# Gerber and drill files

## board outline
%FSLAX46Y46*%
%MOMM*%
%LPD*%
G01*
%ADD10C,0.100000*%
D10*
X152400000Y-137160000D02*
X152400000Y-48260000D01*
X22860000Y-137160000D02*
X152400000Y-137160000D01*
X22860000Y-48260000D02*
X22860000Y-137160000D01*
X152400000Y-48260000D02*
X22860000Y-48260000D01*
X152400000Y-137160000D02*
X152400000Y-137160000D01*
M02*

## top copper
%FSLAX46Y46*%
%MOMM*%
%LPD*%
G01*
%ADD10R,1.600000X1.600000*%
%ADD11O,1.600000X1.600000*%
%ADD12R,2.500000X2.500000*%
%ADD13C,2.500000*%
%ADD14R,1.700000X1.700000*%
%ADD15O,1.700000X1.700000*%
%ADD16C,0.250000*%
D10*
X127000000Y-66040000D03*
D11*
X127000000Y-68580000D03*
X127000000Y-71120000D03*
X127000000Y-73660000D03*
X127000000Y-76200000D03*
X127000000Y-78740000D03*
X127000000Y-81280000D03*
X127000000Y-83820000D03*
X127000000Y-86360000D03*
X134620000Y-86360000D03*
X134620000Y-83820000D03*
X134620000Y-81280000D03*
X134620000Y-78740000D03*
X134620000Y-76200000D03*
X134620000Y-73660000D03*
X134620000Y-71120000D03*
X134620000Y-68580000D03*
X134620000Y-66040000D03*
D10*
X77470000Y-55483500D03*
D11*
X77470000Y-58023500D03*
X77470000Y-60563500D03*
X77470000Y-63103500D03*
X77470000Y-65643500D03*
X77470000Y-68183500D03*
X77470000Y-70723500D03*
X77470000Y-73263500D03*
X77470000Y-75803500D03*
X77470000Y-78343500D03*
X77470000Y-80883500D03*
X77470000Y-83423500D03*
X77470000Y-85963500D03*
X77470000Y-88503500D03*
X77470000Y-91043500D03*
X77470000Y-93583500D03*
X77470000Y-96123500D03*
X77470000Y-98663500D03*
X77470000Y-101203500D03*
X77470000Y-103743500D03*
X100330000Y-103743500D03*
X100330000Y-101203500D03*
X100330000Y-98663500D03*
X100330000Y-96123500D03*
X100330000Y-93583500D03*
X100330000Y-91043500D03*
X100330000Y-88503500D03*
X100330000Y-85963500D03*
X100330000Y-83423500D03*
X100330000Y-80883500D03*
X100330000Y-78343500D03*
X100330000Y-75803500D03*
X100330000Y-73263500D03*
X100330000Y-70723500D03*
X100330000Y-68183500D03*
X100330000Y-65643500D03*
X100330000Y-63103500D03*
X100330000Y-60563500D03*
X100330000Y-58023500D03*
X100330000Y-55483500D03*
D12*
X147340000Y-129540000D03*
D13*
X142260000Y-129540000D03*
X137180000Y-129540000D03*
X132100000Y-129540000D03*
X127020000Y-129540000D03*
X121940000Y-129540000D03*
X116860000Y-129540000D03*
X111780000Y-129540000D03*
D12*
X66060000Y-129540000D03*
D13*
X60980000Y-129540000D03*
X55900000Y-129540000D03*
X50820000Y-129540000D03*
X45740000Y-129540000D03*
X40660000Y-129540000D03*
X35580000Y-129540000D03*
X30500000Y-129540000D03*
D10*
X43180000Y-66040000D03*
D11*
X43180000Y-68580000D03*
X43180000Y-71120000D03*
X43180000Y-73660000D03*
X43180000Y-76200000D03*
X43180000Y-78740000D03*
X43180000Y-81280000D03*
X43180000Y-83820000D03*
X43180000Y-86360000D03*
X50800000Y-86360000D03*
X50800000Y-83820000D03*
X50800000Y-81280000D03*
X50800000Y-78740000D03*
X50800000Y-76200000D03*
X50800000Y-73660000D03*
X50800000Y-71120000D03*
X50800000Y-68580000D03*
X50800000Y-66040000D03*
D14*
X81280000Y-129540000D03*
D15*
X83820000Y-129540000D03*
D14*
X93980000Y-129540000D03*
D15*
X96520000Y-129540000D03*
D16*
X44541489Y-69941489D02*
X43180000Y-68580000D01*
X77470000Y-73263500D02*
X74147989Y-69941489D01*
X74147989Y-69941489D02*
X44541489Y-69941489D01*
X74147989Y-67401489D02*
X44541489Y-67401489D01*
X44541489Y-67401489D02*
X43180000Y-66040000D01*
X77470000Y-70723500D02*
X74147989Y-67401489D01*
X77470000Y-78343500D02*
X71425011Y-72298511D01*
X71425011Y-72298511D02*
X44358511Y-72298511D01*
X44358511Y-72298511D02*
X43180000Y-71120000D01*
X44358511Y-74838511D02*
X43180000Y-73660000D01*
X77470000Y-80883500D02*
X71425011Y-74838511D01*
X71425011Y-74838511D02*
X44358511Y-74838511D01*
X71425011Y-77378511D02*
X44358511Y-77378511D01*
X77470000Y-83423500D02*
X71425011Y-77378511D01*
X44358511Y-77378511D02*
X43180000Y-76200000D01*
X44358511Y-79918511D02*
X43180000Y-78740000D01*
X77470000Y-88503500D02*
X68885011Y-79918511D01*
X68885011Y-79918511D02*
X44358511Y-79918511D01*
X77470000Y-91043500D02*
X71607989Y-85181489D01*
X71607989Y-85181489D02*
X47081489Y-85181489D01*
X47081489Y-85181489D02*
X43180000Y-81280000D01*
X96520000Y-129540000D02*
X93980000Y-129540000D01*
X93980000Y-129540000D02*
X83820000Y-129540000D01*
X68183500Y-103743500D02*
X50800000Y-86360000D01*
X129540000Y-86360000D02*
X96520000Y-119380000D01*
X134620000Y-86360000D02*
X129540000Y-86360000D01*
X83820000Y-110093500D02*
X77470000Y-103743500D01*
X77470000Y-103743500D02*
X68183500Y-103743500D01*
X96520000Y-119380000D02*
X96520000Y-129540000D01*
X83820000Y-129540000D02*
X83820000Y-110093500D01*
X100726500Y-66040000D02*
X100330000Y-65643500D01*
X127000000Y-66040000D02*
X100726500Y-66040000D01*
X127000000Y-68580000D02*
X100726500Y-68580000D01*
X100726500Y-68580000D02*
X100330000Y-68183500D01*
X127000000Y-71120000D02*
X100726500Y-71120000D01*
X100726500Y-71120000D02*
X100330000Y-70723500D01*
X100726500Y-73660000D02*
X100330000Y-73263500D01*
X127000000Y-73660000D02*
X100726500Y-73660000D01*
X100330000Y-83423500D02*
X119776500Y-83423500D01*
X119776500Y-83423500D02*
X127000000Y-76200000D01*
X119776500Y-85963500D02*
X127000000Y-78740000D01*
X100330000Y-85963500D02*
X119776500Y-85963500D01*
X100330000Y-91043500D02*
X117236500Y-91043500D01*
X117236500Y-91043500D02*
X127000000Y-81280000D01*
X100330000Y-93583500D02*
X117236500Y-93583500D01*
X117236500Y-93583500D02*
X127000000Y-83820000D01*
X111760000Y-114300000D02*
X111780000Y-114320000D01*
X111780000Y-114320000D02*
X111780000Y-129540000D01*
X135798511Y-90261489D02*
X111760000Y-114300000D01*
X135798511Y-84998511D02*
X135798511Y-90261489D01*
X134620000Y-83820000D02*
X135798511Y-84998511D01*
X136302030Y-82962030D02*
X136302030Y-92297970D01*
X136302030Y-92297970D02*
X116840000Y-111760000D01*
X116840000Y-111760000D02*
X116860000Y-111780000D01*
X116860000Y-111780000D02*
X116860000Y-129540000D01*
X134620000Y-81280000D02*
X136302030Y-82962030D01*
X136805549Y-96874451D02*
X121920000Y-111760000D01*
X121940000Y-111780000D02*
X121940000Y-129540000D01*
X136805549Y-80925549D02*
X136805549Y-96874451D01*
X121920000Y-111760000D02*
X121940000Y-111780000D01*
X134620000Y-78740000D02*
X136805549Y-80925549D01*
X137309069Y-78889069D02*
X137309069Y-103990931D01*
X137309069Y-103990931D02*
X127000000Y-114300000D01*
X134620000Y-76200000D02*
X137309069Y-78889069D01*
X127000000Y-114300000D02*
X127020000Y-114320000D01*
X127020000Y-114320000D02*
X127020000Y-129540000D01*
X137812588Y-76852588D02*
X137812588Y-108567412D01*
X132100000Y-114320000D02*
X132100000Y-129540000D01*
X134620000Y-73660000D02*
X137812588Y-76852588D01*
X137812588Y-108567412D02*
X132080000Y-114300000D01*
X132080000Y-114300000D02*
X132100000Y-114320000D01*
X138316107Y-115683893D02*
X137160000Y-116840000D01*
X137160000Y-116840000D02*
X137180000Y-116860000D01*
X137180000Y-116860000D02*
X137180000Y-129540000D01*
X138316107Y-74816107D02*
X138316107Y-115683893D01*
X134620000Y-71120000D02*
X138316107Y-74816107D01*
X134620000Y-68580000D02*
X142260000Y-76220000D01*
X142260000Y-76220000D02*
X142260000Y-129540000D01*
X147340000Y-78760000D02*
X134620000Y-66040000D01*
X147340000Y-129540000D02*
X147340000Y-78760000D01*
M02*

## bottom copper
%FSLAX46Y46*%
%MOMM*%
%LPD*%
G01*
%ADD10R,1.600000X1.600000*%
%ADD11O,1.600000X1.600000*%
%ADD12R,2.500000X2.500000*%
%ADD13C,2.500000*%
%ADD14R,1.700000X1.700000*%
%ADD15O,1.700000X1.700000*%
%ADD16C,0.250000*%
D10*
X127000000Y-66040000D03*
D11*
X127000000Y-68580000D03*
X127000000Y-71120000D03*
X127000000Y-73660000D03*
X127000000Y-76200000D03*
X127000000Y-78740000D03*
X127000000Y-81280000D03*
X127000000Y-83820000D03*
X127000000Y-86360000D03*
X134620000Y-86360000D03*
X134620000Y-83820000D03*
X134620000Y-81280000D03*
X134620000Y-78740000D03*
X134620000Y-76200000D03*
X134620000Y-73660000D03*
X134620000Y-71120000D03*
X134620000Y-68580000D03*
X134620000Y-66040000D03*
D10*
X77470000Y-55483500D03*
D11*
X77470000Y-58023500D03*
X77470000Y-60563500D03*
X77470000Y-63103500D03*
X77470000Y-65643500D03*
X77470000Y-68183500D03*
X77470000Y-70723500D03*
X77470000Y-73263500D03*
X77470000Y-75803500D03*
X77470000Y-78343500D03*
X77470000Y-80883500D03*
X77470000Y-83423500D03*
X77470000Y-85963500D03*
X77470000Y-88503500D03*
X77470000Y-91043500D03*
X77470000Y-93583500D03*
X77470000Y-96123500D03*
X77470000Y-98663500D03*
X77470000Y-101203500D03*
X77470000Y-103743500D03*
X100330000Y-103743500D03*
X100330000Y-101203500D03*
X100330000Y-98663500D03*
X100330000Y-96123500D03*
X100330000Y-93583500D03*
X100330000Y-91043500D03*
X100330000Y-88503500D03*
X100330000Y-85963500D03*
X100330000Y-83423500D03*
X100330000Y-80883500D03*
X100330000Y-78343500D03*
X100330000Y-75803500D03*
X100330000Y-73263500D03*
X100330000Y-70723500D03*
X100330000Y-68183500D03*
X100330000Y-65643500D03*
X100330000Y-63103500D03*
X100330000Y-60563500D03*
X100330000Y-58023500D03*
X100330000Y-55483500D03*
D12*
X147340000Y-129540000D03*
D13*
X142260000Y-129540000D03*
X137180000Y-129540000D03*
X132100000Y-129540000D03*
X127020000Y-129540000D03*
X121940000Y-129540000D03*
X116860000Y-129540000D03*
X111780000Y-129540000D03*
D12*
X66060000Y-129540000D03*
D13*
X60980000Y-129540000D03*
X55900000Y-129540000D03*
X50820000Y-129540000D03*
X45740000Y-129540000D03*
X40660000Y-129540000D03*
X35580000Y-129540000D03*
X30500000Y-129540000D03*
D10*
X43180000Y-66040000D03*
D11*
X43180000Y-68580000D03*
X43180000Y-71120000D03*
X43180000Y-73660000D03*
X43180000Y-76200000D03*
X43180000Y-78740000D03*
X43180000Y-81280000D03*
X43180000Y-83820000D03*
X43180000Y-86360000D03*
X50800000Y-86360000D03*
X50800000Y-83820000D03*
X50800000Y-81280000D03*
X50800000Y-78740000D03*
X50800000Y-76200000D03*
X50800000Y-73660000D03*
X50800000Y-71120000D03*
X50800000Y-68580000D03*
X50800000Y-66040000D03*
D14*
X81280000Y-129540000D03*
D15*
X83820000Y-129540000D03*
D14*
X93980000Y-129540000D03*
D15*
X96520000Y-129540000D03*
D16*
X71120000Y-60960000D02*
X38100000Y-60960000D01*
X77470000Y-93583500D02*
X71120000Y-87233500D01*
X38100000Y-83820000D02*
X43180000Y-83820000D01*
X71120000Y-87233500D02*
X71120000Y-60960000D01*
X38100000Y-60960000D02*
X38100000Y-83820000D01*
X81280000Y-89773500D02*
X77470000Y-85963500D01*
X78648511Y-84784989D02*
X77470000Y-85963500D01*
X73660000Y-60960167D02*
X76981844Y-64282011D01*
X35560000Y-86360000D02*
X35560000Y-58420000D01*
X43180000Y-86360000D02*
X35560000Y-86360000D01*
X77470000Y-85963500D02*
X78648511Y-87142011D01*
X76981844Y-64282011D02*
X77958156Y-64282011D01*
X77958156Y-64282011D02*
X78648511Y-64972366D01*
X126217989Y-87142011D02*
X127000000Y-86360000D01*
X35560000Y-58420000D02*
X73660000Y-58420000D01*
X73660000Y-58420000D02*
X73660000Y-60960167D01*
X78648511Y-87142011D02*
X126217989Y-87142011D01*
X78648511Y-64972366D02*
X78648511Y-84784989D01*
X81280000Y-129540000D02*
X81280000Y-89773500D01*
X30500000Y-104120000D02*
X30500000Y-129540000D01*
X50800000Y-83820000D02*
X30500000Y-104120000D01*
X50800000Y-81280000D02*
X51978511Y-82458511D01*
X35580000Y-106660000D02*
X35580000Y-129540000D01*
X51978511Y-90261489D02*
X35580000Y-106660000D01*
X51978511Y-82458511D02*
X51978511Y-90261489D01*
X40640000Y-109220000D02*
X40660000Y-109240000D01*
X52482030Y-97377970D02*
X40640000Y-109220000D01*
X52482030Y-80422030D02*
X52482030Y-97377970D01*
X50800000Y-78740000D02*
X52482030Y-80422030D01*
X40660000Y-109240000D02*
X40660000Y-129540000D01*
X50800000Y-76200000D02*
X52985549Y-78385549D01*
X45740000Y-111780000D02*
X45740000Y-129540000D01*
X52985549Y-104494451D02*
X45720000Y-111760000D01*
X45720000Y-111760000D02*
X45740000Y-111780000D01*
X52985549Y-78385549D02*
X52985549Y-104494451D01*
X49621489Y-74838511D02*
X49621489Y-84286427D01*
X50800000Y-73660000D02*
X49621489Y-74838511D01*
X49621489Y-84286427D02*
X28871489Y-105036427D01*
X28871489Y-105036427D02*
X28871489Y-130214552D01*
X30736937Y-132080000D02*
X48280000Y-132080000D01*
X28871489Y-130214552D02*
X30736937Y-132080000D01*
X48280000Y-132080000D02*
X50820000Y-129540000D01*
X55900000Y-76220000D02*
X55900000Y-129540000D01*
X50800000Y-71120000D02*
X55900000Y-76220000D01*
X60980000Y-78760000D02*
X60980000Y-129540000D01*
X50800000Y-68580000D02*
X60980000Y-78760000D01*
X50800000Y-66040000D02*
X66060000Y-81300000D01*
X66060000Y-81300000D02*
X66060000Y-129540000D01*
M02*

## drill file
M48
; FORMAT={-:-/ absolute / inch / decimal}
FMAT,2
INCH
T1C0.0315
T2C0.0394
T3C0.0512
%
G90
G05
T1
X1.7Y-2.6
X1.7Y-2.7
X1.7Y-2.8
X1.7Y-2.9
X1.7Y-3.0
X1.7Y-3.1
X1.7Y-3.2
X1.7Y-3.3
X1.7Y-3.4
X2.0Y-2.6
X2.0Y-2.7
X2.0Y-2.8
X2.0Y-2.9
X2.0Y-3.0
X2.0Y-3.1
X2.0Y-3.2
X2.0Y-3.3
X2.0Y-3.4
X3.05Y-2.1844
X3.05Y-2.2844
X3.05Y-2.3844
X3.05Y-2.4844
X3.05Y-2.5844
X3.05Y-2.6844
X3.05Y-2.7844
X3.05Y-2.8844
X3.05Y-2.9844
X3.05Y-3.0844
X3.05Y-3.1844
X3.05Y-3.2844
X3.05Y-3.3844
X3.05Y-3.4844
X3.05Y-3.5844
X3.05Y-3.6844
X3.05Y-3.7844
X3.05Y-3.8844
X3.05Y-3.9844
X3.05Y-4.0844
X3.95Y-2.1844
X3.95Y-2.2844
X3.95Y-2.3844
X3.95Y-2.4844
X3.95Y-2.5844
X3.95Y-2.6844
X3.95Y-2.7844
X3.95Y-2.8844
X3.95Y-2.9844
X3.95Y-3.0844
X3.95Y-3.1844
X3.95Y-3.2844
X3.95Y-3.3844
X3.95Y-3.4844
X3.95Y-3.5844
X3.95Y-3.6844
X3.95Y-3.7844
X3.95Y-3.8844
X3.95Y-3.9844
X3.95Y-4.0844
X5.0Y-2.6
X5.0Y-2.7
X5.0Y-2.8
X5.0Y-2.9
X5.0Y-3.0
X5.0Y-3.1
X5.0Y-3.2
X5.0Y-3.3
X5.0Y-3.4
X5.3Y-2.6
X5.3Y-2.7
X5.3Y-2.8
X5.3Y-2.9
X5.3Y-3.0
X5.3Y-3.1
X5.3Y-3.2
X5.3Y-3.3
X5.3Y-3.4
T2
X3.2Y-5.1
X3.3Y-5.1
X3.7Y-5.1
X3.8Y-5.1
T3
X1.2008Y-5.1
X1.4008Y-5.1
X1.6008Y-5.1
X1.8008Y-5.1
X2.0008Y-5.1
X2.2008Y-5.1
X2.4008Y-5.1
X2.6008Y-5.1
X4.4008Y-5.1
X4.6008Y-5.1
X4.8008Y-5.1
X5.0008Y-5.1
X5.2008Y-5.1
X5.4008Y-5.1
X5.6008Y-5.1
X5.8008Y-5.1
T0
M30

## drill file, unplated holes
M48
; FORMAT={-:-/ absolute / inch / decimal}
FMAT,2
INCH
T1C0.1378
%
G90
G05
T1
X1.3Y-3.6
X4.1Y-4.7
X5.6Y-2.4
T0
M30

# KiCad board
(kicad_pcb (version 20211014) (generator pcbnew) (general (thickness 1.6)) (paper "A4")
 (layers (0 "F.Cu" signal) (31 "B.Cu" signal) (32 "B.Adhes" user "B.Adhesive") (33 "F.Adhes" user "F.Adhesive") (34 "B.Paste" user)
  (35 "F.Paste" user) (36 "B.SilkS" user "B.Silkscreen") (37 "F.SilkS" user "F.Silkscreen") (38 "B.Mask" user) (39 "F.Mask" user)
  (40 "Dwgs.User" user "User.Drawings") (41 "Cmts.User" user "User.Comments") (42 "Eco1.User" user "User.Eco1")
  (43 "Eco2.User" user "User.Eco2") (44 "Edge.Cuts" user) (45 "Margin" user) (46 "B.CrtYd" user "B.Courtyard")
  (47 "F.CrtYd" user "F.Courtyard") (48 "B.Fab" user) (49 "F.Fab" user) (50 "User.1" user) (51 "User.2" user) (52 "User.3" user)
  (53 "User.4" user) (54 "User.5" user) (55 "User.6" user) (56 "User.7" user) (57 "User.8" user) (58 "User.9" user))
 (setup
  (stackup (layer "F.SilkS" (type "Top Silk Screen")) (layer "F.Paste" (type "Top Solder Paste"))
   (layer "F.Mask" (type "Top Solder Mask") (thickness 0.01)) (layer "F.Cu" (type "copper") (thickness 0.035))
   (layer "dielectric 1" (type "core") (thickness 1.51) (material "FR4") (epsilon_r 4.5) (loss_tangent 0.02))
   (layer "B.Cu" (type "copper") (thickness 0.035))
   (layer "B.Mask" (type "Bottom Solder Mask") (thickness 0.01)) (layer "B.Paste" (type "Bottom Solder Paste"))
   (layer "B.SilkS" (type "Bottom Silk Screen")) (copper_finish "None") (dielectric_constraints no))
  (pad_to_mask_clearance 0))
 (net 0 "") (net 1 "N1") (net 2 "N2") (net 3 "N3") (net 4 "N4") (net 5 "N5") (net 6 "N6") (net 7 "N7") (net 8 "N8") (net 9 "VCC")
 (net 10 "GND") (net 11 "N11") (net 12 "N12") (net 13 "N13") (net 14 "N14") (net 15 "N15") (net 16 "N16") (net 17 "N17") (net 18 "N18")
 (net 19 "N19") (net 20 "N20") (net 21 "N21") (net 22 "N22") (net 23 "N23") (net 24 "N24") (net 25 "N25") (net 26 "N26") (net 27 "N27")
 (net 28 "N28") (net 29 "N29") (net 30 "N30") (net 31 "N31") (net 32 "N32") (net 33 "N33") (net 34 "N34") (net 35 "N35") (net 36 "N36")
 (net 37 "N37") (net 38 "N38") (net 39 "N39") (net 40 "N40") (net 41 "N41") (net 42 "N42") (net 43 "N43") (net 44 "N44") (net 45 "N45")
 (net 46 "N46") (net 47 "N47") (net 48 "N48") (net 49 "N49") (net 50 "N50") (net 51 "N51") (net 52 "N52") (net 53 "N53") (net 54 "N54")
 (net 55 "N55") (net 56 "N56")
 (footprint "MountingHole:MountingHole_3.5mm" (layer "F.Cu") (at 142.24 60.96)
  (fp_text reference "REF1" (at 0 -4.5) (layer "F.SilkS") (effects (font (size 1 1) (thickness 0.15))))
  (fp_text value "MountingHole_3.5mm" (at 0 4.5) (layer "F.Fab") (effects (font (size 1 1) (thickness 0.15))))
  (pad "" np_thru_hole circle (at 0 0) (size 3.5 3.5) (drill 3.5) (layers *.Cu *.Mask)))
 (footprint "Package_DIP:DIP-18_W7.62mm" (layer "F.Cu") (at 127 66.04)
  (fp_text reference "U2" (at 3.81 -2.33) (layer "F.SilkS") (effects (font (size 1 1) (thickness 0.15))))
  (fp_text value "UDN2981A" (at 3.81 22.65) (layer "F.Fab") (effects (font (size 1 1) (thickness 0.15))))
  (pad "1" thru_hole rect (at 0 0) (size 1.6 1.6) (drill 0.8) (layers *.Cu *.Mask) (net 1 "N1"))
  (pad "2" thru_hole oval (at 0 2.54) (size 1.6 1.6) (drill 0.8) (layers *.Cu *.Mask) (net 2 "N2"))
  (pad "3" thru_hole oval (at 0 5.08) (size 1.6 1.6) (drill 0.8) (layers *.Cu *.Mask) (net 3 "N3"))
  (pad "4" thru_hole oval (at 0 7.62) (size 1.6 1.6) (drill 0.8) (layers *.Cu *.Mask) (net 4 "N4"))
  (pad "5" thru_hole oval (at 0 10.16) (size 1.6 1.6) (drill 0.8) (layers *.Cu *.Mask) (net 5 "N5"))
  (pad "6" thru_hole oval (at 0 12.7) (size 1.6 1.6) (drill 0.8) (layers *.Cu *.Mask) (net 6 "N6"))
  (pad "7" thru_hole oval (at 0 15.24) (size 1.6 1.6) (drill 0.8) (layers *.Cu *.Mask) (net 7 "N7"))
  (pad "8" thru_hole oval (at 0 17.78) (size 1.6 1.6) (drill 0.8) (layers *.Cu *.Mask) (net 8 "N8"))
  (pad "9" thru_hole oval (at 0 20.32) (size 1.6 1.6) (drill 0.8) (layers *.Cu *.Mask) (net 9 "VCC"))
  (pad "10" thru_hole oval (at 7.62 20.32) (size 1.6 1.6) (drill 0.8) (layers *.Cu *.Mask) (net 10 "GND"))
  (pad "11" thru_hole oval (at 7.62 17.78) (size 1.6 1.6) (drill 0.8) (layers *.Cu *.Mask) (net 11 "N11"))
  (pad "12" thru_hole oval (at 7.62 15.24) (size 1.6 1.6) (drill 0.8) (layers *.Cu *.Mask) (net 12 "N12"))
  (pad "13" thru_hole oval (at 7.62 12.7) (size 1.6 1.6) (drill 0.8) (layers *.Cu *.Mask) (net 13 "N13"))
  (pad "14" thru_hole oval (at 7.62 10.16) (size 1.6 1.6) (drill 0.8) (layers *.Cu *.Mask) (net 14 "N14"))
  (pad "15" thru_hole oval (at 7.62 7.62) (size 1.6 1.6) (drill 0.8) (layers *.Cu *.Mask) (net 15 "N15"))
  (pad "16" thru_hole oval (at 7.62 5.08) (size 1.6 1.6) (drill 0.8) (layers *.Cu *.Mask) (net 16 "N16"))
  (pad "17" thru_hole oval (at 7.62 2.54) (size 1.6 1.6) (drill 0.8) (layers *.Cu *.Mask) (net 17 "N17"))
  (pad "18" thru_hole oval (at 7.62 0) (size 1.6 1.6) (drill 0.8) (layers *.Cu *.Mask) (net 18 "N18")))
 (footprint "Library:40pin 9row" (layer "F.Cu") (at 77.47 55.4835)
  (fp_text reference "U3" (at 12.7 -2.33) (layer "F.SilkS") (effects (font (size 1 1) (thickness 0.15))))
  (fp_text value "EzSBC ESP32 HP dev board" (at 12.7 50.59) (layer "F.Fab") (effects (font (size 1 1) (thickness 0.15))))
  (pad "1" thru_hole rect (at 0 0) (size 1.6 1.6) (drill 0.8) (layers *.Cu *.Mask) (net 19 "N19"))
  (pad "2" thru_hole oval (at 0 2.54) (size 1.6 1.6) (drill 0.8) (layers *.Cu *.Mask) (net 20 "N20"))
  (pad "3" thru_hole oval (at 0 5.08) (size 1.6 1.6) (drill 0.8) (layers *.Cu *.Mask) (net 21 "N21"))
  (pad "4" thru_hole oval (at 0 7.62) (size 1.6 1.6) (drill 0.8) (layers *.Cu *.Mask) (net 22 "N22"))
  (pad "5" thru_hole oval (at 0 10.16) (size 1.6 1.6) (drill 0.8) (layers *.Cu *.Mask) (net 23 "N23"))
  (pad "6" thru_hole oval (at 0 12.7) (size 1.6 1.6) (drill 0.8) (layers *.Cu *.Mask) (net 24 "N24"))
  (pad "7" thru_hole oval (at 0 15.24) (size 1.6 1.6) (drill 0.8) (layers *.Cu *.Mask) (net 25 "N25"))
  (pad "8" thru_hole oval (at 0 17.78) (size 1.6 1.6) (drill 0.8) (layers *.Cu *.Mask) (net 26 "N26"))
  (pad "9" thru_hole oval (at 0 20.32) (size 1.6 1.6) (drill 0.8) (layers *.Cu *.Mask) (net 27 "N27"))
  (pad "10" thru_hole oval (at 0 22.86) (size 1.6 1.6) (drill 0.8) (layers *.Cu *.Mask) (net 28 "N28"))
  (pad "11" thru_hole oval (at 0 25.4) (size 1.6 1.6) (drill 0.8) (layers *.Cu *.Mask) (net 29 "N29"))
  (pad "12" thru_hole oval (at 0 27.94) (size 1.6 1.6) (drill 0.8) (layers *.Cu *.Mask) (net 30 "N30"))
  (pad "13" thru_hole oval (at 0 30.48) (size 1.6 1.6) (drill 0.8) (layers *.Cu *.Mask) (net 9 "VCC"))
  (pad "14" thru_hole oval (at 0 33.02) (size 1.6 1.6) (drill 0.8) (layers *.Cu *.Mask) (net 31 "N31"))
  (pad "15" thru_hole oval (at 0 35.56) (size 1.6 1.6) (drill 0.8) (layers *.Cu *.Mask) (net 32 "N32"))
  (pad "16" thru_hole oval (at 0 38.1) (size 1.6 1.6) (drill 0.8) (layers *.Cu *.Mask) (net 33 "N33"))
  (pad "17" thru_hole oval (at 0 40.64) (size 1.6 1.6) (drill 0.8) (layers *.Cu *.Mask) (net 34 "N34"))
  (pad "18" thru_hole oval (at 0 43.18) (size 1.6 1.6) (drill 0.8) (layers *.Cu *.Mask) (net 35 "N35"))
  (pad "19" thru_hole oval (at 0 45.72) (size 1.6 1.6) (drill 0.8) (layers *.Cu *.Mask) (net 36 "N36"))
  (pad "20" thru_hole oval (at 0 48.26) (size 1.6 1.6) (drill 0.8) (layers *.Cu *.Mask) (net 10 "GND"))
  (pad "21" thru_hole oval (at 22.86 48.26) (size 1.6 1.6) (drill 0.8) (layers *.Cu *.Mask) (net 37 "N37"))
  (pad "22" thru_hole oval (at 22.86 45.72) (size 1.6 1.6) (drill 0.8) (layers *.Cu *.Mask) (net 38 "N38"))
  (pad "23" thru_hole oval (at 22.86 43.18) (size 1.6 1.6) (drill 0.8) (layers *.Cu *.Mask) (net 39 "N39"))
  (pad "24" thru_hole oval (at 22.86 40.64) (size 1.6 1.6) (drill 0.8) (layers *.Cu *.Mask) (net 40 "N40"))
  (pad "25" thru_hole oval (at 22.86 38.1) (size 1.6 1.6) (drill 0.8) (layers *.Cu *.Mask) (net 8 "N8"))
  (pad "26" thru_hole oval (at 22.86 35.56) (size 1.6 1.6) (drill 0.8) (layers *.Cu *.Mask) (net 7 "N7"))
  (pad "27" thru_hole oval (at 22.86 33.02) (size 1.6 1.6) (drill 0.8) (layers *.Cu *.Mask) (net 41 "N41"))
  (pad "28" thru_hole oval (at 22.86 30.48) (size 1.6 1.6) (drill 0.8) (layers *.Cu *.Mask) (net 6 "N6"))
  (pad "29" thru_hole oval (at 22.86 27.94) (size 1.6 1.6) (drill 0.8) (layers *.Cu *.Mask) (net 5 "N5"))
  (pad "30" thru_hole oval (at 22.86 25.4) (size 1.6 1.6) (drill 0.8) (layers *.Cu *.Mask) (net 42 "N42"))
  (pad "31" thru_hole oval (at 22.86 22.86) (size 1.6 1.6) (drill 0.8) (layers *.Cu *.Mask) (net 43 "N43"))
  (pad "32" thru_hole oval (at 22.86 20.32) (size 1.6 1.6) (drill 0.8) (layers *.Cu *.Mask) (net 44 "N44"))
  (pad "33" thru_hole oval (at 22.86 17.78) (size 1.6 1.6) (drill 0.8) (layers *.Cu *.Mask) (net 4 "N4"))
  (pad "34" thru_hole oval (at 22.86 15.24) (size 1.6 1.6) (drill 0.8) (layers *.Cu *.Mask) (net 3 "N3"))
  (pad "35" thru_hole oval (at 22.86 12.7) (size 1.6 1.6) (drill 0.8) (layers *.Cu *.Mask) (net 2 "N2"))
  (pad "36" thru_hole oval (at 22.86 10.16) (size 1.6 1.6) (drill 0.8) (layers *.Cu *.Mask) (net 1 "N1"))
  (pad "37" thru_hole oval (at 22.86 7.62) (size 1.6 1.6) (drill 0.8) (layers *.Cu *.Mask) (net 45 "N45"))
  (pad "38" thru_hole oval (at 22.86 5.08) (size 1.6 1.6) (drill 0.8) (layers *.Cu *.Mask) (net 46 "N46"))
  (pad "39" thru_hole oval (at 22.86 2.54) (size 1.6 1.6) (drill 0.8) (layers *.Cu *.Mask) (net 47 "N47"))
  (pad "40" thru_hole oval (at 22.86 0) (size 1.6 1.6) (drill 0.8) (layers *.Cu *.Mask) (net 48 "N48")))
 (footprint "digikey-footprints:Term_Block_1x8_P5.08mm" (layer "F.Cu") (at 147.34 129.54 180)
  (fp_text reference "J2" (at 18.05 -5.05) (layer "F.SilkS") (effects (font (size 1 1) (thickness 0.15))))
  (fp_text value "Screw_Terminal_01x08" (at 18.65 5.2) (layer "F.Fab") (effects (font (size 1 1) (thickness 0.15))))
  (pad "1" thru_hole rect locked (at 0 0 180) (size 2.5 2.5) (drill 1.3) (layers *.Cu *.Mask) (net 18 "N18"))
  (pad "2" thru_hole circle locked (at 5.08 0 180) (size 2.5 2.5) (drill 1.3) (layers *.Cu *.Mask) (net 17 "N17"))
  (pad "3" thru_hole circle locked (at 10.16 0 180) (size 2.5 2.5) (drill 1.3) (layers *.Cu *.Mask) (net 16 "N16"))
  (pad "4" thru_hole circle locked (at 15.24 0 180) (size 2.5 2.5) (drill 1.3) (layers *.Cu *.Mask) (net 15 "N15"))
  (pad "5" thru_hole circle locked (at 20.32 0 180) (size 2.5 2.5) (drill 1.3) (layers *.Cu *.Mask) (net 14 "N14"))
  (pad "6" thru_hole circle locked (at 25.4 0 180) (size 2.5 2.5) (drill 1.3) (layers *.Cu *.Mask) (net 13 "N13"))
  (pad "7" thru_hole circle locked (at 30.48 0 180) (size 2.5 2.5) (drill 1.3) (layers *.Cu *.Mask) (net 12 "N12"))
  (pad "8" thru_hole circle locked (at 35.56 0 180) (size 2.5 2.5) (drill 1.3) (layers *.Cu *.Mask) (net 11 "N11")))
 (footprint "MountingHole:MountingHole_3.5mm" (layer "F.Cu") (at 104.14 119.38)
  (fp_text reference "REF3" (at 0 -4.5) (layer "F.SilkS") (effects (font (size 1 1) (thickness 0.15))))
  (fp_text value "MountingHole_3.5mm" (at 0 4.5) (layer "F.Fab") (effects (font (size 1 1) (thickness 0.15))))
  (pad "" np_thru_hole circle (at 0 0) (size 3.5 3.5) (drill 3.5) (layers *.Cu *.Mask)))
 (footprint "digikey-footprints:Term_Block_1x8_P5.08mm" (layer "F.Cu") (at 66.06 129.54 180)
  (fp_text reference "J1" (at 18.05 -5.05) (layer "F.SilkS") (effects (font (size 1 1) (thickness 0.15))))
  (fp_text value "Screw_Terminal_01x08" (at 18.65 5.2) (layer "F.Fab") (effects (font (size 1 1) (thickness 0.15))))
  (pad "1" thru_hole rect locked (at 0 0 180) (size 2.5 2.5) (drill 1.3) (layers *.Cu *.Mask) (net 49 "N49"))
  (pad "2" thru_hole circle locked (at 5.08 0 180) (size 2.5 2.5) (drill 1.3) (layers *.Cu *.Mask) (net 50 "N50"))
  (pad "3" thru_hole circle locked (at 10.16 0 180) (size 2.5 2.5) (drill 1.3) (layers *.Cu *.Mask) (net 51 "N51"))
  (pad "4" thru_hole circle locked (at 15.24 0 180) (size 2.5 2.5) (drill 1.3) (layers *.Cu *.Mask) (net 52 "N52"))
  (pad "5" thru_hole circle locked (at 20.32 0 180) (size 2.5 2.5) (drill 1.3) (layers *.Cu *.Mask) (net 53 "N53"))
  (pad "6" thru_hole circle locked (at 25.4 0 180) (size 2.5 2.5) (drill 1.3) (layers *.Cu *.Mask) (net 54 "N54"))
  (pad "7" thru_hole circle locked (at 30.48 0 180) (size 2.5 2.5) (drill 1.3) (layers *.Cu *.Mask) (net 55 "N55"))
  (pad "8" thru_hole circle locked (at 35.56 0 180) (size 2.5 2.5) (drill 1.3) (layers *.Cu *.Mask) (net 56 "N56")))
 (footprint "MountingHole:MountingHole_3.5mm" (layer "F.Cu") (at 33.02 91.44)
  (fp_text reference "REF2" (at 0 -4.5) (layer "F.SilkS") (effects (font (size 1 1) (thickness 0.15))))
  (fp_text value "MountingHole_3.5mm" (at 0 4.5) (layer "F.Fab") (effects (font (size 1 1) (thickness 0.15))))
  (pad "" np_thru_hole circle (at 0 0) (size 3.5 3.5) (drill 3.5) (layers *.Cu *.Mask)))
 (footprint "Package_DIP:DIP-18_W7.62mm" (layer "F.Cu") (at 43.18 66.04)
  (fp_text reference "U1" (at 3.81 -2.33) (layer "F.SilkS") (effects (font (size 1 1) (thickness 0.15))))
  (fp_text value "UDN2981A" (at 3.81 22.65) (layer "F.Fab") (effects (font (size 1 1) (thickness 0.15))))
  (pad "1" thru_hole rect (at 0 0) (size 1.6 1.6) (drill 0.8) (layers *.Cu *.Mask) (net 25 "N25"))
  (pad "2" thru_hole oval (at 0 2.54) (size 1.6 1.6) (drill 0.8) (layers *.Cu *.Mask) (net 26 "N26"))
  (pad "3" thru_hole oval (at 0 5.08) (size 1.6 1.6) (drill 0.8) (layers *.Cu *.Mask) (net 28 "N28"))
  (pad "4" thru_hole oval (at 0 7.62) (size 1.6 1.6) (drill 0.8) (layers *.Cu *.Mask) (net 29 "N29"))
  (pad "5" thru_hole oval (at 0 10.16) (size 1.6 1.6) (drill 0.8) (layers *.Cu *.Mask) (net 30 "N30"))
  (pad "6" thru_hole oval (at 0 12.7) (size 1.6 1.6) (drill 0.8) (layers *.Cu *.Mask) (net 31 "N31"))
  (pad "7" thru_hole oval (at 0 15.24) (size 1.6 1.6) (drill 0.8) (layers *.Cu *.Mask) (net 32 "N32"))
  (pad "8" thru_hole oval (at 0 17.78) (size 1.6 1.6) (drill 0.8) (layers *.Cu *.Mask) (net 33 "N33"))
  (pad "9" thru_hole oval (at 0 20.32) (size 1.6 1.6) (drill 0.8) (layers *.Cu *.Mask) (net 9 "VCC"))
  (pad "10" thru_hole oval (at 7.62 20.32) (size 1.6 1.6) (drill 0.8) (layers *.Cu *.Mask) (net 10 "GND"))
  (pad "11" thru_hole oval (at 7.62 17.78) (size 1.6 1.6) (drill 0.8) (layers *.Cu *.Mask) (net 56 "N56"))
  (pad "12" thru_hole oval (at 7.62 15.24) (size 1.6 1.6) (drill 0.8) (layers *.Cu *.Mask) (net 55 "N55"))
  (pad "13" thru_hole oval (at 7.62 12.7) (size 1.6 1.6) (drill 0.8) (layers *.Cu *.Mask) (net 54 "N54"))
  (pad "14" thru_hole oval (at 7.62 10.16) (size 1.6 1.6) (drill 0.8) (layers *.Cu *.Mask) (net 53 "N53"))
  (pad "15" thru_hole oval (at 7.62 7.62) (size 1.6 1.6) (drill 0.8) (layers *.Cu *.Mask) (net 52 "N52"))
  (pad "16" thru_hole oval (at 7.62 5.08) (size 1.6 1.6) (drill 0.8) (layers *.Cu *.Mask) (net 51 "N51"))
  (pad "17" thru_hole oval (at 7.62 2.54) (size 1.6 1.6) (drill 0.8) (layers *.Cu *.Mask) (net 50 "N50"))
  (pad "18" thru_hole oval (at 7.62 0) (size 1.6 1.6) (drill 0.8) (layers *.Cu *.Mask) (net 49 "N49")))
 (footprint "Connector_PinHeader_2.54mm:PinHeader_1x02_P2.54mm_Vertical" (layer "F.Cu") (at 81.28 129.54 90)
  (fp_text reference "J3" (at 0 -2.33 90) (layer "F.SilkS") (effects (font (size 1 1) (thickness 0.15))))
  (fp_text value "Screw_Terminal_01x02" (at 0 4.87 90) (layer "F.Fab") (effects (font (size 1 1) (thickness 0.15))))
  (pad "1" thru_hole rect (at 0 0 90) (size 1.7 1.7) (drill 1) (layers *.Cu *.Mask) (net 9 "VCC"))
  (pad "2" thru_hole oval (at 0 2.54 90) (size 1.7 1.7) (drill 1) (layers *.Cu *.Mask) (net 10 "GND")))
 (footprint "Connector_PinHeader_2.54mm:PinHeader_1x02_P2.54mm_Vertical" (layer "F.Cu") (at 93.98 129.54 90)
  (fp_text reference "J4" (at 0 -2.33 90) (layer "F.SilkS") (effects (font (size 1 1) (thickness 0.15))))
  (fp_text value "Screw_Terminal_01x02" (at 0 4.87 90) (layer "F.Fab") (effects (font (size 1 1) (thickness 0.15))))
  (pad "1" thru_hole rect (at 0 0 90) (size 1.7 1.7) (drill 1) (layers *.Cu *.Mask) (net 10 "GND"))
  (pad "2" thru_hole oval (at 0 2.54 90) (size 1.7 1.7) (drill 1) (layers *.Cu *.Mask) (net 10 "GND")))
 (gr_line (start 152.4 137.16) (end 152.4 48.26) (layer "Edge.Cuts") (width 0.1))
 (gr_line (start 22.86 137.16) (end 152.4 137.16) (layer "Edge.Cuts") (width 0.1))
 (gr_line (start 22.86 48.26) (end 22.86 137.16) (layer "Edge.Cuts") (width 0.1))
 (gr_line (start 152.4 48.26) (end 22.86 48.26) (layer "Edge.Cuts") (width 0.1))
 (gr_line (start 152.4 137.16) (end 152.4 137.16) (layer "Edge.Cuts") (width 0.1))
 (segment (start 74.147989 67.401489) (end 44.541489 67.401489) (width 0.25) (layer "F.Cu") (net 25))
 (segment (start 44.541489 67.401489) (end 43.18 66.04) (width 0.25) (layer "F.Cu") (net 25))
 (segment (start 77.47 70.7235) (end 74.147989 67.401489) (width 0.25) (layer "F.Cu") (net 25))
 (segment (start 44.541489 69.941489) (end 43.18 68.58) (width 0.25) (layer "F.Cu") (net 26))
 (segment (start 74.147989 69.941489) (end 44.541489 69.941489) (width 0.25) (layer "F.Cu") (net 26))
 (segment (start 77.47 73.2635) (end 74.147989 69.941489) (width 0.25) (layer "F.Cu") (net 26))
 (segment (start 77.47 78.3435) (end 71.425011 72.298511) (width 0.25) (layer "F.Cu") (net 28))
 (segment (start 71.425011 72.298511) (end 44.358511 72.298511) (width 0.25) (layer "F.Cu") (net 28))
 (segment (start 44.358511 72.298511) (end 43.18 71.12) (width 0.25) (layer "F.Cu") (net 28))
 (segment (start 44.358511 74.838511) (end 43.18 73.66) (width 0.25) (layer "F.Cu") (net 29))
 (segment (start 77.47 80.8835) (end 71.425011 74.838511) (width 0.25) (layer "F.Cu") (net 29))
 (segment (start 71.425011 74.838511) (end 44.358511 74.838511) (width 0.25) (layer "F.Cu") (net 29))
 (segment (start 71.425011 77.378511) (end 44.358511 77.378511) (width 0.25) (layer "F.Cu") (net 30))
 (segment (start 77.47 83.4235) (end 71.425011 77.378511) (width 0.25) (layer "F.Cu") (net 30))
 (segment (start 44.358511 77.378511) (end 43.18 76.2) (width 0.25) (layer "F.Cu") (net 30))
 (segment (start 44.358511 79.918511) (end 43.18 78.74) (width 0.25) (layer "F.Cu") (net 31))
 (segment (start 77.47 88.5035) (end 68.885011 79.918511) (width 0.25) (layer "F.Cu") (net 31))
 (segment (start 68.885011 79.918511) (end 44.358511 79.918511) (width 0.25) (layer "F.Cu") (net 31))
 (segment (start 77.47 91.0435) (end 71.607989 85.181489) (width 0.25) (layer "F.Cu") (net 32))
 (segment (start 71.607989 85.181489) (end 47.081489 85.181489) (width 0.25) (layer "F.Cu") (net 32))
 (segment (start 47.081489 85.181489) (end 43.18 81.28) (width 0.25) (layer "F.Cu") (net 32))
 (segment (start 71.12 60.96) (end 38.1 60.96) (width 0.25) (layer "B.Cu") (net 33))
 (segment (start 77.47 93.5835) (end 71.12 87.2335) (width 0.25) (layer "B.Cu") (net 33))
 (segment (start 38.1 83.82) (end 43.18 83.82) (width 0.25) (layer "B.Cu") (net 33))
 (segment (start 71.12 87.2335) (end 71.12 60.96) (width 0.25) (layer "B.Cu") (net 33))
 (segment (start 38.1 60.96) (end 38.1 83.82) (width 0.25) (layer "B.Cu") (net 33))
 (segment (start 81.28 89.7735) (end 77.47 85.9635) (width 0.25) (layer "B.Cu") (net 9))
 (segment (start 78.648511 84.784989) (end 77.47 85.9635) (width 0.25) (layer "B.Cu") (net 9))
 (segment (start 73.66 60.960167) (end 76.981844 64.282011) (width 0.25) (layer "B.Cu") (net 9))
 (segment (start 35.56 86.36) (end 35.56 58.42) (width 0.25) (layer "B.Cu") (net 9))
 (segment (start 43.18 86.36) (end 35.56 86.36) (width 0.25) (layer "B.Cu") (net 9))
 (segment (start 77.47 85.9635) (end 78.648511 87.142011) (width 0.25) (layer "B.Cu") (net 9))
 (segment (start 76.981844 64.282011) (end 77.958156 64.282011) (width 0.25) (layer "B.Cu") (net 9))
 (segment (start 77.958156 64.282011) (end 78.648511 64.972366) (width 0.25) (layer "B.Cu") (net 9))
 (segment (start 126.217989 87.142011) (end 127 86.36) (width 0.25) (layer "B.Cu") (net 9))
 (segment (start 35.56 58.42) (end 73.66 58.42) (width 0.25) (layer "B.Cu") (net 9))
 (segment (start 73.66 58.42) (end 73.66 60.960167) (width 0.25) (layer "B.Cu") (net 9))
 (segment (start 78.648511 87.142011) (end 126.217989 87.142011) (width 0.25) (layer "B.Cu") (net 9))
 (segment (start 78.648511 64.972366) (end 78.648511 84.784989) (width 0.25) (layer "B.Cu") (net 9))
 (segment (start 81.28 129.54) (end 81.28 89.7735) (width 0.25) (layer "B.Cu") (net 9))
 (segment (start 96.52 129.54) (end 93.98 129.54) (width 0.25) (layer "F.Cu") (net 10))
 (segment (start 93.98 129.54) (end 83.82 129.54) (width 0.25) (layer "F.Cu") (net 10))
 (segment (start 68.1835 103.7435) (end 50.8 86.36) (width 0.25) (layer "F.Cu") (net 10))
 (segment (start 129.54 86.36) (end 96.52 119.38) (width 0.25) (layer "F.Cu") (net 10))
 (segment (start 134.62 86.36) (end 129.54 86.36) (width 0.25) (layer "F.Cu") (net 10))
 (segment (start 83.82 110.0935) (end 77.47 103.7435) (width 0.25) (layer "F.Cu") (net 10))
 (segment (start 77.47 103.7435) (end 68.1835 103.7435) (width 0.25) (layer "F.Cu") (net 10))
 (segment (start 96.52 119.38) (end 96.52 129.54) (width 0.25) (layer "F.Cu") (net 10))
 (segment (start 83.82 129.54) (end 83.82 110.0935) (width 0.25) (layer "F.Cu") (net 10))
 (segment (start 30.5 104.12) (end 30.5 129.54) (width 0.25) (layer "B.Cu") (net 56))
 (segment (start 50.8 83.82) (end 30.5 104.12) (width 0.25) (layer "B.Cu") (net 56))
 (segment (start 50.8 81.28) (end 51.978511 82.458511) (width 0.25) (layer "B.Cu") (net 55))
 (segment (start 35.58 106.66) (end 35.58 129.54) (width 0.25) (layer "B.Cu") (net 55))
 (segment (start 51.978511 90.261489) (end 35.58 106.66) (width 0.25) (layer "B.Cu") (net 55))
 (segment (start 51.978511 82.458511) (end 51.978511 90.261489) (width 0.25) (layer "B.Cu") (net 55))
 (segment (start 40.64 109.22) (end 40.66 109.24) (width 0.25) (layer "B.Cu") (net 54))
 (segment (start 52.48203 97.37797) (end 40.64 109.22) (width 0.25) (layer "B.Cu") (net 54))
 (segment (start 52.48203 80.42203) (end 52.48203 97.37797) (width 0.25) (layer "B.Cu") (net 54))
 (segment (start 50.8 78.74) (end 52.48203 80.42203) (width 0.25) (layer "B.Cu") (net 54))
 (segment (start 40.66 109.24) (end 40.66 129.54) (width 0.25) (layer "B.Cu") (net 54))
 (segment (start 50.8 76.2) (end 52.985549 78.385549) (width 0.25) (layer "B.Cu") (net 53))
 (segment (start 45.74 111.78) (end 45.74 129.54) (width 0.25) (layer "B.Cu") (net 53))
 (segment (start 52.985549 104.494451) (end 45.72 111.76) (width 0.25) (layer "B.Cu") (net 53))
 (segment (start 45.72 111.76) (end 45.74 111.78) (width 0.25) (layer "B.Cu") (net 53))
 (segment (start 52.985549 78.385549) (end 52.985549 104.494451) (width 0.25) (layer "B.Cu") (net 53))
 (segment (start 49.621489 74.838511) (end 49.621489 84.286427) (width 0.25) (layer "B.Cu") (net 52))
 (segment (start 50.8 73.66) (end 49.621489 74.838511) (width 0.25) (layer "B.Cu") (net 52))
 (segment (start 49.621489 84.286427) (end 28.871489 105.036427) (width 0.25) (layer "B.Cu") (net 52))
 (segment (start 28.871489 105.036427) (end 28.871489 130.214552) (width 0.25) (layer "B.Cu") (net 52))
 (segment (start 30.736937 132.08) (end 48.28 132.08) (width 0.25) (layer "B.Cu") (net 52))
 (segment (start 28.871489 130.214552) (end 30.736937 132.08) (width 0.25) (layer "B.Cu") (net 52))
 (segment (start 48.28 132.08) (end 50.82 129.54) (width 0.25) (layer "B.Cu") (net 52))
 (segment (start 55.9 76.22) (end 55.9 129.54) (width 0.25) (layer "B.Cu") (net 51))
 (segment (start 50.8 71.12) (end 55.9 76.22) (width 0.25) (layer "B.Cu") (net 51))
 (segment (start 60.98 78.76) (end 60.98 129.54) (width 0.25) (layer "B.Cu") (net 50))
 (segment (start 50.8 68.58) (end 60.98 78.76) (width 0.25) (layer "B.Cu") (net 50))
 (segment (start 50.8 66.04) (end 66.06 81.3) (width 0.25) (layer "B.Cu") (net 49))
 (segment (start 66.06 81.3) (end 66.06 129.54) (width 0.25) (layer "B.Cu") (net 49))
 (segment (start 100.7265 66.04) (end 100.33 65.6435) (width 0.25) (layer "F.Cu") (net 1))
 (segment (start 127 66.04) (end 100.7265 66.04) (width 0.25) (layer "F.Cu") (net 1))
 (segment (start 127 68.58) (end 100.7265 68.58) (width 0.25) (layer "F.Cu") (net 2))
 (segment (start 100.7265 68.58) (end 100.33 68.1835) (width 0.25) (layer "F.Cu") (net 2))
 (segment (start 127 71.12) (end 100.7265 71.12) (width 0.25) (layer "F.Cu") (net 3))
 (segment (start 100.7265 71.12) (end 100.33 70.7235) (width 0.25) (layer "F.Cu") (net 3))
 (segment (start 100.7265 73.66) (end 100.33 73.2635) (width 0.25) (layer "F.Cu") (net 4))
 (segment (start 127 73.66) (end 100.7265 73.66) (width 0.25) (layer "F.Cu") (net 4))
 (segment (start 100.33 83.4235) (end 119.7765 83.4235) (width 0.25) (layer "F.Cu") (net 5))
 (segment (start 119.7765 83.4235) (end 127 76.2) (width 0.25) (layer "F.Cu") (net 5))
 (segment (start 119.7765 85.9635) (end 127 78.74) (width 0.25) (layer "F.Cu") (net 6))
 (segment (start 100.33 85.9635) (end 119.7765 85.9635) (width 0.25) (layer "F.Cu") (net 6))
 (segment (start 100.33 91.0435) (end 117.2365 91.0435) (width 0.25) (layer "F.Cu") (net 7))
 (segment (start 117.2365 91.0435) (end 127 81.28) (width 0.25) (layer "F.Cu") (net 7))
 (segment (start 100.33 93.5835) (end 117.2365 93.5835) (width 0.25) (layer "F.Cu") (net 8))
 (segment (start 117.2365 93.5835) (end 127 83.82) (width 0.25) (layer "F.Cu") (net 8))
 (segment (start 111.76 114.3) (end 111.78 114.32) (width 0.25) (layer "F.Cu") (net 11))
 (segment (start 111.78 114.32) (end 111.78 129.54) (width 0.25) (layer "F.Cu") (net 11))
 (segment (start 135.798511 90.261489) (end 111.76 114.3) (width 0.25) (layer "F.Cu") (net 11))
 (segment (start 135.798511 84.998511) (end 135.798511 90.261489) (width 0.25) (layer "F.Cu") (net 11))
 (segment (start 134.62 83.82) (end 135.798511 84.998511) (width 0.25) (layer "F.Cu") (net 11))
 (segment (start 136.30203 82.96203) (end 136.30203 92.29797) (width 0.25) (layer "F.Cu") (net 12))
 (segment (start 136.30203 92.29797) (end 116.84 111.76) (width 0.25) (layer "F.Cu") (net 12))
 (segment (start 116.84 111.76) (end 116.86 111.78) (width 0.25) (layer "F.Cu") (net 12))
 (segment (start 116.86 111.78) (end 116.86 129.54) (width 0.25) (layer "F.Cu") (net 12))
 (segment (start 134.62 81.28) (end 136.30203 82.96203) (width 0.25) (layer "F.Cu") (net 12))
 (segment (start 136.805549 96.874451) (end 121.92 111.76) (width 0.25) (layer "F.Cu") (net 13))
 (segment (start 121.94 111.78) (end 121.94 129.54) (width 0.25) (layer "F.Cu") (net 13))
 (segment (start 136.805549 80.925549) (end 136.805549 96.874451) (width 0.25) (layer "F.Cu") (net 13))
 (segment (start 121.92 111.76) (end 121.94 111.78) (width 0.25) (layer "F.Cu") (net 13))
 (segment (start 134.62 78.74) (end 136.805549 80.925549) (width 0.25) (layer "F.Cu") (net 13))
 (segment (start 137.309069 78.889069) (end 137.309069 103.990931) (width 0.25) (layer "F.Cu") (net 14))
 (segment (start 137.309069 103.990931) (end 127 114.3) (width 0.25) (layer "F.Cu") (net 14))
 (segment (start 134.62 76.2) (end 137.309069 78.889069) (width 0.25) (layer "F.Cu") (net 14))
 (segment (start 127 114.3) (end 127.02 114.32) (width 0.25) (layer "F.Cu") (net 14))
 (segment (start 127.02 114.32) (end 127.02 129.54) (width 0.25) (layer "F.Cu") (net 14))
 (segment (start 137.812588 76.852588) (end 137.812588 108.567412) (width 0.25) (layer "F.Cu") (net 15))
 (segment (start 132.1 114.32) (end 132.1 129.54) (width 0.25) (layer "F.Cu") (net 15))
 (segment (start 134.62 73.66) (end 137.812588 76.852588) (width 0.25) (layer "F.Cu") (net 15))
 (segment (start 137.812588 108.567412) (end 132.08 114.3) (width 0.25) (layer "F.Cu") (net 15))
 (segment (start 132.08 114.3) (end 132.1 114.32) (width 0.25) (layer "F.Cu") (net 15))
 (segment (start 138.316107 115.683893) (end 137.16 116.84) (width 0.25) (layer "F.Cu") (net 16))
 (segment (start 137.16 116.84) (end 137.18 116.86) (width 0.25) (layer "F.Cu") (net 16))
 (segment (start 137.18 116.86) (end 137.18 129.54) (width 0.25) (layer "F.Cu") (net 16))
 (segment (start 138.316107 74.816107) (end 138.316107 115.683893) (width 0.25) (layer "F.Cu") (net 16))
 (segment (start 134.62 71.12) (end 138.316107 74.816107) (width 0.25) (layer "F.Cu") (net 16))
 (segment (start 134.62 68.58) (end 142.26 76.22) (width 0.25) (layer "F.Cu") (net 17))
 (segment (start 142.26 76.22) (end 142.26 129.54) (width 0.25) (layer "F.Cu") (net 17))
 (segment (start 147.34 78.76) (end 134.62 66.04) (width 0.25) (layer "F.Cu") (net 18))
 (segment (start 147.34 129.54) (end 147.34 78.76) (width 0.25) (layer "F.Cu") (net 18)))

